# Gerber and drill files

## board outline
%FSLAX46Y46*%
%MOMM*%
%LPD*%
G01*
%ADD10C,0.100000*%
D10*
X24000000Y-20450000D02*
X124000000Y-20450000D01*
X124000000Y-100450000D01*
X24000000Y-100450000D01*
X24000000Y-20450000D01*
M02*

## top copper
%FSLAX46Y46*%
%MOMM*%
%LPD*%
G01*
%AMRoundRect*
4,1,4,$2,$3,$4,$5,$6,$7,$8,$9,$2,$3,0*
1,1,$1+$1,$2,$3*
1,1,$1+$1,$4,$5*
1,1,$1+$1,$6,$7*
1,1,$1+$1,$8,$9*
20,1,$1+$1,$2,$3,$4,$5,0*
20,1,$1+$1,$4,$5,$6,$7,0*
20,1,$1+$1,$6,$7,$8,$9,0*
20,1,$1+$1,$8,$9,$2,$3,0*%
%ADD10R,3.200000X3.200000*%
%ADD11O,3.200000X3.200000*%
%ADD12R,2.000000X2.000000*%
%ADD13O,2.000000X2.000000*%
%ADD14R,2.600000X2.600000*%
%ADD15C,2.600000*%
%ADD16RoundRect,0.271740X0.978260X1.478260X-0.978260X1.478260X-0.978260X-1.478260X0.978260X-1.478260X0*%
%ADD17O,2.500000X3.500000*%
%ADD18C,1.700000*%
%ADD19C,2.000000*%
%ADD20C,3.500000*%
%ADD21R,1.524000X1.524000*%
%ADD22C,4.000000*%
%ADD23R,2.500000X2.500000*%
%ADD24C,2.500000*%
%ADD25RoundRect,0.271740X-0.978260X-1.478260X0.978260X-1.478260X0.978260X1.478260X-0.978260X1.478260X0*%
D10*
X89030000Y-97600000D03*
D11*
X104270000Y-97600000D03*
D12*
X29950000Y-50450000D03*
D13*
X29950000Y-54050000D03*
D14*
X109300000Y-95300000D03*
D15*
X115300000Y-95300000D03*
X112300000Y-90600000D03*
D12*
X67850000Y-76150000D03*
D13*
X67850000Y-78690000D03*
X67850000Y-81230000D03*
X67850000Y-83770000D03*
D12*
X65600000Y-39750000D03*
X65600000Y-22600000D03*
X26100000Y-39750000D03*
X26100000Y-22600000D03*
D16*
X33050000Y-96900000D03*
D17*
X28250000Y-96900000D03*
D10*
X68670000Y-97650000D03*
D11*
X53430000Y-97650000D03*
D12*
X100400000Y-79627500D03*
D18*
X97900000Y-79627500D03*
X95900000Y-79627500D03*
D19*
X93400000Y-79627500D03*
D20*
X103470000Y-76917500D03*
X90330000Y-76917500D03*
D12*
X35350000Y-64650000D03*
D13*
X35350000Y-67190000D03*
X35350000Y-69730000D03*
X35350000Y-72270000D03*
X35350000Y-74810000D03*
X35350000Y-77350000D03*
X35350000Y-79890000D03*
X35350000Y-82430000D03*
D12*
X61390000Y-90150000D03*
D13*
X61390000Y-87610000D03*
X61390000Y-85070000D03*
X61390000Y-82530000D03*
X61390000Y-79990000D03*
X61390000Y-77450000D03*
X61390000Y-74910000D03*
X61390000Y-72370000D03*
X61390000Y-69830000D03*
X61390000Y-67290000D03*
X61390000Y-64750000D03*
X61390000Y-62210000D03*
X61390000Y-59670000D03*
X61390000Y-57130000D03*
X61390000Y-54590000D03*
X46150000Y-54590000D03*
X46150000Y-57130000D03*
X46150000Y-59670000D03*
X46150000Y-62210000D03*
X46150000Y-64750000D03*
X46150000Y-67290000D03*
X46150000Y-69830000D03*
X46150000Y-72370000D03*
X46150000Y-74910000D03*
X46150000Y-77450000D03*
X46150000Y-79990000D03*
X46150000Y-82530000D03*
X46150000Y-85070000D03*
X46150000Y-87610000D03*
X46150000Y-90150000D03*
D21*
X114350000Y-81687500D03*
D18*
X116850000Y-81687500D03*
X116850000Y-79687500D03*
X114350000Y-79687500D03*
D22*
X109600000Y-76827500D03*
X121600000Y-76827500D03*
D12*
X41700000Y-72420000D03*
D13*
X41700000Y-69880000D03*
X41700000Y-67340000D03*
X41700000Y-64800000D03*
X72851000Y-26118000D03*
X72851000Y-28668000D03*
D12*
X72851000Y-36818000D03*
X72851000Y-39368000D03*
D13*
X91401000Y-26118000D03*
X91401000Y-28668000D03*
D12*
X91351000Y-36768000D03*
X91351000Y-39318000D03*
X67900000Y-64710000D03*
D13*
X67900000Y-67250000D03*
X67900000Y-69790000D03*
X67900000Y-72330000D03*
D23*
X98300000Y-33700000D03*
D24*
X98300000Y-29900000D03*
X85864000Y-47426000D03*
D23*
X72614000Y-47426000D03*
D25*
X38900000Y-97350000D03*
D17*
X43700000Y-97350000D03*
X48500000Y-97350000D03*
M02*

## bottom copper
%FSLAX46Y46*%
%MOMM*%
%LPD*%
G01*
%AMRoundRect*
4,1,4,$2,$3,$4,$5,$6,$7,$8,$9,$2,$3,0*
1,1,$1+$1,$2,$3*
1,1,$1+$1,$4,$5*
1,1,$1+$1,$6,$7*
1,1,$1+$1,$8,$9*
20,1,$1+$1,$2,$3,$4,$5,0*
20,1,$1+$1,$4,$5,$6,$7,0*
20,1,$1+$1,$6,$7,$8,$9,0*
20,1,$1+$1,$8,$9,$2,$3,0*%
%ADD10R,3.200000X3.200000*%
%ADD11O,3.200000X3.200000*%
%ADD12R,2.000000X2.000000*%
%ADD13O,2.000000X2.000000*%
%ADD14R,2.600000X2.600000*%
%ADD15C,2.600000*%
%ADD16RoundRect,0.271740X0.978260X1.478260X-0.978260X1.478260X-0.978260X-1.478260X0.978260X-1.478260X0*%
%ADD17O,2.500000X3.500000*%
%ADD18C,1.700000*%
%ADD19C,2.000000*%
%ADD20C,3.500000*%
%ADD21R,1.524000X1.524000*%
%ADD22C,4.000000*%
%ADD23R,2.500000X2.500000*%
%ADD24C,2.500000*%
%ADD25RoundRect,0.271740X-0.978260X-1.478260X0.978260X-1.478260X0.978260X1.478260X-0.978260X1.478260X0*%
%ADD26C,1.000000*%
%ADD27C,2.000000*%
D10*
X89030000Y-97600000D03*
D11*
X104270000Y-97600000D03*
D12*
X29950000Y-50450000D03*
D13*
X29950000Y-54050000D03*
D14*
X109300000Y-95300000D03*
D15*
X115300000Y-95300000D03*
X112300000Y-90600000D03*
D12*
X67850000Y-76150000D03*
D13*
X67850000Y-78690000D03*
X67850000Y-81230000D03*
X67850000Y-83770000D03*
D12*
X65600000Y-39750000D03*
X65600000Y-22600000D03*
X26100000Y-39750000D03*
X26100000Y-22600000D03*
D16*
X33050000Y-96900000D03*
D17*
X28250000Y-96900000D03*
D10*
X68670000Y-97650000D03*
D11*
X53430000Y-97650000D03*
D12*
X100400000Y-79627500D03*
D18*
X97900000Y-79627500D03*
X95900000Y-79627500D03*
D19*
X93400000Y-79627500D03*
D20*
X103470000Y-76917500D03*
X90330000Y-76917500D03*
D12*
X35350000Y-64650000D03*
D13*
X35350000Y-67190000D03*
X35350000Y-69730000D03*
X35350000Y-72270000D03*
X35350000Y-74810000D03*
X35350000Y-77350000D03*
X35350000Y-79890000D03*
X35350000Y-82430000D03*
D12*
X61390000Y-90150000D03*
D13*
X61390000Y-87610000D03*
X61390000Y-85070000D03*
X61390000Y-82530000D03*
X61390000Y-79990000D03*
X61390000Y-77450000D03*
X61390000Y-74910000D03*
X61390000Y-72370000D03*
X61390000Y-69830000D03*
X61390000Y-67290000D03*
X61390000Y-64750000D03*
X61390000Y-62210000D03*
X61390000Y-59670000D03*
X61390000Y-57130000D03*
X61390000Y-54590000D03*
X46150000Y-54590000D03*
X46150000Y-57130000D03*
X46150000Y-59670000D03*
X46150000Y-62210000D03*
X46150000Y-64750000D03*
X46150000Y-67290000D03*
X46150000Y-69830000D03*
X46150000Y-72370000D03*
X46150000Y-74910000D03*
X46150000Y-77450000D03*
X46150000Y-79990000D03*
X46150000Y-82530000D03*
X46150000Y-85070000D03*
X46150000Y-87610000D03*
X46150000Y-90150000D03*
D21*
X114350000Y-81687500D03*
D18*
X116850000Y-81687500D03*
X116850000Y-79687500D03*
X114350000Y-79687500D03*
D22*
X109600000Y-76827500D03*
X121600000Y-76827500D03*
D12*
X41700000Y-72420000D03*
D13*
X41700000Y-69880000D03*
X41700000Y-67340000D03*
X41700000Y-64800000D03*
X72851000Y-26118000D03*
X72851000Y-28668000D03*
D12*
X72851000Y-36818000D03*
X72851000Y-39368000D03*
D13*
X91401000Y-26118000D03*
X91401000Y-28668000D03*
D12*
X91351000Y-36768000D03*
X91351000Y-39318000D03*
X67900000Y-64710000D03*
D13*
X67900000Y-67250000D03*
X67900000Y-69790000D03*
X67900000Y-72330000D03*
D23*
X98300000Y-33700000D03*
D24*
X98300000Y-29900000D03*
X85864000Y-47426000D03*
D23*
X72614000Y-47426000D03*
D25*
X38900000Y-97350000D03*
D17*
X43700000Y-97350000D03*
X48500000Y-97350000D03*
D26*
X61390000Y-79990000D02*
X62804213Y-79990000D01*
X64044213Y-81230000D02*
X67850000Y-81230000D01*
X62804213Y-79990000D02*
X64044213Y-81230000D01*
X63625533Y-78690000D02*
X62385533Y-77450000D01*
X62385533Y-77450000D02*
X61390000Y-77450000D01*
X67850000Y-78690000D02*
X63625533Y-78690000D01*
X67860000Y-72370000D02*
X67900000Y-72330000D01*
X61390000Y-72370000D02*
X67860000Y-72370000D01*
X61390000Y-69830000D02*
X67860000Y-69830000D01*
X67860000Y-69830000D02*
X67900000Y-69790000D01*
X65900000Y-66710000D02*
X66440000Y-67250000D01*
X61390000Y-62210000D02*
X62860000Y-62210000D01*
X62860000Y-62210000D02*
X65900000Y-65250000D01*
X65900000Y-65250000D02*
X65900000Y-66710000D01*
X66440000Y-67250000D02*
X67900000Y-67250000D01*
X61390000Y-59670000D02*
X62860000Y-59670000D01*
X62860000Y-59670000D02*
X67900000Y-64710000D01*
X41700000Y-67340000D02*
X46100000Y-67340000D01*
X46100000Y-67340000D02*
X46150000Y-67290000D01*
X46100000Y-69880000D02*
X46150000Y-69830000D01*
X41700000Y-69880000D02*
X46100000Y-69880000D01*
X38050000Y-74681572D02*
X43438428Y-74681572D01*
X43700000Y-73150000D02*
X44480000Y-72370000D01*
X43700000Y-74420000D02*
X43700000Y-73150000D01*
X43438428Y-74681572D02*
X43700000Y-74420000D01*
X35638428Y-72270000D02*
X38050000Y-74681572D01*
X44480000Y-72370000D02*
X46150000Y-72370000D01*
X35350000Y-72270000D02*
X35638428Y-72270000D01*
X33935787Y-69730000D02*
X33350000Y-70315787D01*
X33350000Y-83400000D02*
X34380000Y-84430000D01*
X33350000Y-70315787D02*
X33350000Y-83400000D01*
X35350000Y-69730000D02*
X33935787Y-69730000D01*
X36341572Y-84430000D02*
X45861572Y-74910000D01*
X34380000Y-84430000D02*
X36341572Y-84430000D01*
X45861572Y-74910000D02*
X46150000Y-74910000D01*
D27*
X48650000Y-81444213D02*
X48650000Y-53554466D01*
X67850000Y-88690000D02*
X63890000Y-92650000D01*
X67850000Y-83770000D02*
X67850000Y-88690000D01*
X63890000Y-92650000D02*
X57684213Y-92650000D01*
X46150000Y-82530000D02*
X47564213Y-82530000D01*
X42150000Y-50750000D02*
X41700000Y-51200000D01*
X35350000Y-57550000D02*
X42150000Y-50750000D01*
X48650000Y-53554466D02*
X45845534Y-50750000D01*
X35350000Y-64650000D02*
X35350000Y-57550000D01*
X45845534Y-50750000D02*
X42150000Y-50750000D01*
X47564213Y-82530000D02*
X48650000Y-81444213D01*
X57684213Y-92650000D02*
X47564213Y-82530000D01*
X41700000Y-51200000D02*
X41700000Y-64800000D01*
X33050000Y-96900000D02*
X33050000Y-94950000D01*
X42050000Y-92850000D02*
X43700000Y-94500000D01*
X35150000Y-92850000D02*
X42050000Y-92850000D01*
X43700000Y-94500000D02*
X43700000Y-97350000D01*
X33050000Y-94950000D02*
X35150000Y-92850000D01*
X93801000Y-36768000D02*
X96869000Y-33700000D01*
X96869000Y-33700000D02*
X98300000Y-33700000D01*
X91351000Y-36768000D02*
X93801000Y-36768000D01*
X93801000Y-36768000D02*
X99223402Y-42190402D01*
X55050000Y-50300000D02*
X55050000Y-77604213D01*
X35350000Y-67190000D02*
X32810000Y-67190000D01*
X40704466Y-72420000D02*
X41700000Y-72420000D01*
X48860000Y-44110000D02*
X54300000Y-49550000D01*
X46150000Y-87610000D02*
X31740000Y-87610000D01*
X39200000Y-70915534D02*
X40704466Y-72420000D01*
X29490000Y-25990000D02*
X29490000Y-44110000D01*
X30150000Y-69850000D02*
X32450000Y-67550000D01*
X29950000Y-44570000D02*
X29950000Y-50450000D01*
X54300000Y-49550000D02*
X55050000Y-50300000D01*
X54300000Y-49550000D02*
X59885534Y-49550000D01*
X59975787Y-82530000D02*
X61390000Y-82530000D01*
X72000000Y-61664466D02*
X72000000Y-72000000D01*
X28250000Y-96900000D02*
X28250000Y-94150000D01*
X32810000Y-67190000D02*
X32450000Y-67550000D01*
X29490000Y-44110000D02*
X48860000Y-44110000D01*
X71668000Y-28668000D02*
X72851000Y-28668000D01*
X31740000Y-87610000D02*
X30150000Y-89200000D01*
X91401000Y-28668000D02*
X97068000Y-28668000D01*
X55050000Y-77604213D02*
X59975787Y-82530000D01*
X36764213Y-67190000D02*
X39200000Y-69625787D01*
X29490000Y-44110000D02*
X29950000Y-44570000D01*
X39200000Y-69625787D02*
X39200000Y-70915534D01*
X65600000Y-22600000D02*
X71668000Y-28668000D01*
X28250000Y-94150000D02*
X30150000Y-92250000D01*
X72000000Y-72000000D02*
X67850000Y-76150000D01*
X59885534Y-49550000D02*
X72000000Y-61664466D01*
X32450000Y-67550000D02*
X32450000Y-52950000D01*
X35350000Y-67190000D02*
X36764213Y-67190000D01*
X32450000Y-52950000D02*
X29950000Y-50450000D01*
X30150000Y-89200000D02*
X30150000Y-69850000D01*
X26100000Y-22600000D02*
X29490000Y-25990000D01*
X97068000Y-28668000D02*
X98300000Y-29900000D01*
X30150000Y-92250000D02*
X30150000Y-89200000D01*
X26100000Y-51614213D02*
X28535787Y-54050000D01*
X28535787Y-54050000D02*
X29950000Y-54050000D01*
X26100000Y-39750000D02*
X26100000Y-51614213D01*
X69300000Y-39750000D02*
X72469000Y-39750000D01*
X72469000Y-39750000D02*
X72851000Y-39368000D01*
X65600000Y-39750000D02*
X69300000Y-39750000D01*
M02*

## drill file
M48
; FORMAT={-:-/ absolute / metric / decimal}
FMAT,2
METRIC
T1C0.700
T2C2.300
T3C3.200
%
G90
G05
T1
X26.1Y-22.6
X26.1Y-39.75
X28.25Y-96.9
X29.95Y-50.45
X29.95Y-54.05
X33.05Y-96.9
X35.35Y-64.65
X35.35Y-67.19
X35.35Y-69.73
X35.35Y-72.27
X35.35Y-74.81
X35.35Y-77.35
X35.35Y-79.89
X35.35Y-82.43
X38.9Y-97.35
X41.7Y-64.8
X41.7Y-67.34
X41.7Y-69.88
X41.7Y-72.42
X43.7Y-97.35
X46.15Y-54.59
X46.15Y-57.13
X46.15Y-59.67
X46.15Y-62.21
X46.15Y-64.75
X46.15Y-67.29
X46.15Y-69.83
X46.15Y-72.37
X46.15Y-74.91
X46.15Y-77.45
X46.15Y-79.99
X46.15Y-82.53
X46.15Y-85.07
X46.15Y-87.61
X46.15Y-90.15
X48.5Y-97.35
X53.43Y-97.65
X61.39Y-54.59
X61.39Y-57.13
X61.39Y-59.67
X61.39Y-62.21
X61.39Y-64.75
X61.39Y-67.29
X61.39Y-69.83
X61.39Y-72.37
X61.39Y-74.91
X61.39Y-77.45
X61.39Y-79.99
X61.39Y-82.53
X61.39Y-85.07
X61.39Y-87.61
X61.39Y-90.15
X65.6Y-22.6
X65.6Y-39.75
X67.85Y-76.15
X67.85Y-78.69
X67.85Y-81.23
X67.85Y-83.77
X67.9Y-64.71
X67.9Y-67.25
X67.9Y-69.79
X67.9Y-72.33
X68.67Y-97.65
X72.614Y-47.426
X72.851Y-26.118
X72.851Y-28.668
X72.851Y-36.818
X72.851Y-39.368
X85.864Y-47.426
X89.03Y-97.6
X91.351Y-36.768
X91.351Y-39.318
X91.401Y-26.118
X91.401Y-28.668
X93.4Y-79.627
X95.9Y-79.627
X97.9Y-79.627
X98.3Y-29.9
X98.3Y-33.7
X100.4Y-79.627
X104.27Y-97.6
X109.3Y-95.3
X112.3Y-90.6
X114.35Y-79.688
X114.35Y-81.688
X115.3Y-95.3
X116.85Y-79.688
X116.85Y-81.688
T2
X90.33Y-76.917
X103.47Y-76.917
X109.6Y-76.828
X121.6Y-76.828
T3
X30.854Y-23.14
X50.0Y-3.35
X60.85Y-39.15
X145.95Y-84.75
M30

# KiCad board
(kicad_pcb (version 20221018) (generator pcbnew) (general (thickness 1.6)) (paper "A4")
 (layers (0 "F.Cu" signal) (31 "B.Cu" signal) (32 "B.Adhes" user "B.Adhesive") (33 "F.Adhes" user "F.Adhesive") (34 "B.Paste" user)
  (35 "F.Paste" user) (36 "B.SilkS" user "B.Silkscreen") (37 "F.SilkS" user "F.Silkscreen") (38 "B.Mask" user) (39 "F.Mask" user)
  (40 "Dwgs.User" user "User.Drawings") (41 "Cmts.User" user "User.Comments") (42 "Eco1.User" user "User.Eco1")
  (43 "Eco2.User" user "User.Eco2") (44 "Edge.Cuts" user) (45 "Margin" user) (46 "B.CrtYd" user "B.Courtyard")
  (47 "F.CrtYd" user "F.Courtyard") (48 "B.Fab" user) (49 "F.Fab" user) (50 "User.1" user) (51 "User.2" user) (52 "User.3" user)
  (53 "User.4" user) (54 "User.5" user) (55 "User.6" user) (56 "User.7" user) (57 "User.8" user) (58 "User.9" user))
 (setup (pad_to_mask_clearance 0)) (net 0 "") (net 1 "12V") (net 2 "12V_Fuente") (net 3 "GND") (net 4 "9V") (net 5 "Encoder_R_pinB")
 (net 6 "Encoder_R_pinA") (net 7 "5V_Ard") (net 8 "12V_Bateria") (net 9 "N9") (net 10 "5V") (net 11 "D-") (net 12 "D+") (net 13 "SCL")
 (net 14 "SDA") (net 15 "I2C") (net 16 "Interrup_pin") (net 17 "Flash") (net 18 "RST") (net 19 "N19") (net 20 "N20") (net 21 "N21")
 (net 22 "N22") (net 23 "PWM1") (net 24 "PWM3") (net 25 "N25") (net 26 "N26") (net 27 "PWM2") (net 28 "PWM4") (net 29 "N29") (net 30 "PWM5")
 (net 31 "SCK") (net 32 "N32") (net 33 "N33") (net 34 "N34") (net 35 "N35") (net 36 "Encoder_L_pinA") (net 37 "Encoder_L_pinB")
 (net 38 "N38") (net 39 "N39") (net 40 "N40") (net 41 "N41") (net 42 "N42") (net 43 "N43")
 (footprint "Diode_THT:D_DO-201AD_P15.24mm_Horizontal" (layer "F.Cu") (at 89.03 97.6)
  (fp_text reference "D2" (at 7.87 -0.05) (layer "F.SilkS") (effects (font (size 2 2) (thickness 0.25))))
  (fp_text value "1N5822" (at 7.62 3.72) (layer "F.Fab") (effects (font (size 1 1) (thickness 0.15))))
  (pad "1" thru_hole rect (at 0 0) (size 3.2 3.2) (drill 0.7) (layers "*.Cu" "*.Mask") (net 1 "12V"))
  (pad "2" thru_hole oval (at 15.24 0) (size 3.2 3.2) (drill 0.7) (layers "*.Cu" "*.Mask") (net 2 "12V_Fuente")))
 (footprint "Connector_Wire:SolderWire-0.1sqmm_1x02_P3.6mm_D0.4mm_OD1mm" (layer "F.Cu") (at 29.95 50.45 -90)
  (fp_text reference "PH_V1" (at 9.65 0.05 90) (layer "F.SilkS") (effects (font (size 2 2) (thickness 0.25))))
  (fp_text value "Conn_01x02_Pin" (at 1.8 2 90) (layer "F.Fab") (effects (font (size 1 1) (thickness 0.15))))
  (pad "1" thru_hole rect (at 0 0 270) (size 2 2) (drill 0.7) (layers "*.Cu" "*.Mask") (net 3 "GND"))
  (pad "2" thru_hole oval (at 3.6 0 270) (size 2 2) (drill 0.7) (layers "*.Cu" "*.Mask") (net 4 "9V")))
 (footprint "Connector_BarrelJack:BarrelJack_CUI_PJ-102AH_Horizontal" (layer "F.Cu") (at 109.3 95.3 90)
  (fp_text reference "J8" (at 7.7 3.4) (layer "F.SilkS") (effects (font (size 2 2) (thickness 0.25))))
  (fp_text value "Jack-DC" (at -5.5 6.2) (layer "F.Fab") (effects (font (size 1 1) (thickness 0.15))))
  (pad "1" thru_hole rect (at 0 0 90) (size 2.6 2.6) (drill 0.7) (layers "*.Cu" "*.Mask") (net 2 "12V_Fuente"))
  (pad "2" thru_hole circle (at 0 6 90) (size 2.6 2.6) (drill 0.7) (layers "*.Cu" "*.Mask") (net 3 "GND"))
  (pad "3" thru_hole circle (at 4.7 3 90) (size 2.6 2.6) (drill 0.7) (layers "*.Cu" "*.Mask")))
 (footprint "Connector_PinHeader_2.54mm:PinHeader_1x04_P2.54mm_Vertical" (layer "F.Cu") (at 67.85 76.15)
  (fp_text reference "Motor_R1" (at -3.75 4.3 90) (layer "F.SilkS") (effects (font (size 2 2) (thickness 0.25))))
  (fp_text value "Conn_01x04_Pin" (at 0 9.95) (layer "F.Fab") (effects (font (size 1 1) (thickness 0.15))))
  (pad "1" thru_hole rect (at 0 0) (size 2 2) (drill 0.7) (layers "*.Cu" "*.Mask") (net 3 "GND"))
  (pad "2" thru_hole oval (at 0 2.54) (size 2 2) (drill 0.7) (layers "*.Cu" "*.Mask") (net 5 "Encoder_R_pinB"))
  (pad "3" thru_hole oval (at 0 5.08) (size 2 2) (drill 0.7) (layers "*.Cu" "*.Mask") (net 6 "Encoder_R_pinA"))
  (pad "4" thru_hole oval (at 0 7.62) (size 2 2) (drill 0.7) (layers "*.Cu" "*.Mask") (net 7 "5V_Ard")))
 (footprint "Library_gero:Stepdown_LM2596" (layer "F.Cu") (at 67.45 41.7 180)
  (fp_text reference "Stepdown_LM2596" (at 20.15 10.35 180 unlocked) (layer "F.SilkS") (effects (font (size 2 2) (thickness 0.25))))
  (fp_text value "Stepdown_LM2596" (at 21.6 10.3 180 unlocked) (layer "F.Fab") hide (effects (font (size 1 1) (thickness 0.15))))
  (pad "" np_thru_hole circle (at 6.6 2.55 180) (size 3.2 3.2) (drill 3.2) (layers "F&B.Cu" "*.Mask") (thermal_bridge_angle 90))
  (pad "" np_thru_hole circle (at 36.596 18.56 180) (size 3.2 3.2) (drill 3.2) (layers "F&B.Cu" "*.Mask") (thermal_bridge_angle 90))
  (pad "1" thru_hole rect (at 1.85 1.95 180) (size 2 2) (drill 0.7) (layers "*.Cu" "*.Mask") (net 1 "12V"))
  (pad "2" thru_hole rect (at 1.85 19.1 180) (size 2 2) (drill 0.7) (layers "*.Cu" "*.Mask") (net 3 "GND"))
  (pad "3" thru_hole rect (at 41.35 1.95 180) (size 2 2) (drill 0.7) (layers "*.Cu" "*.Mask") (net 4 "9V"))
  (pad "4" thru_hole rect (at 41.35 19.1 180) (size 2 2) (drill 0.7) (layers "*.Cu" "*.Mask") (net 3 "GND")))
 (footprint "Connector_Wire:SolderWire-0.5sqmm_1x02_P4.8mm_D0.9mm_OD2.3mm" (layer "F.Cu") (at 33.05 96.9 180)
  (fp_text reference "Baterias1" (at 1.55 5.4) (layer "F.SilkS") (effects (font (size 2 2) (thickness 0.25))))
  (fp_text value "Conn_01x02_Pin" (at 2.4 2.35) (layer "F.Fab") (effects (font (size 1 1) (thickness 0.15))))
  (pad "1" thru_hole roundrect (at 0 0 180) (size 2.5 3.5) (drill 0.7) (layers "*.Cu" "*.Mask") (roundrect_rratio 0.108696)
   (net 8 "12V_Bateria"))
  (pad "2" thru_hole oval (at 4.8 0 180) (size 2.5 3.5) (drill 0.7) (layers "*.Cu" "*.Mask") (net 3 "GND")))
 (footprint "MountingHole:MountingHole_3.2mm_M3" (layer "F.Cu") (at 50 3.35)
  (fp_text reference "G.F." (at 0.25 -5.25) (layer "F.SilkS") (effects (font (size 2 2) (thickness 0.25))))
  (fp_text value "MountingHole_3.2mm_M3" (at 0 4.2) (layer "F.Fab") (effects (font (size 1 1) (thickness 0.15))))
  (pad "" np_thru_hole circle (at 0 0) (size 3.2 3.2) (drill 3.2) (layers "F&B.Cu" "*.Mask")))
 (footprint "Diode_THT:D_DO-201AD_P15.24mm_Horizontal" (layer "F.Cu") (at 68.67 97.65 180)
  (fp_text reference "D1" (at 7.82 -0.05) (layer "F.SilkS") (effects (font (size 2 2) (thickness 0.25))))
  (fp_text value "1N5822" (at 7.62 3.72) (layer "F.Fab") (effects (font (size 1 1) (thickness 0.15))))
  (pad "1" thru_hole rect (at 0 0 180) (size 3.2 3.2) (drill 0.7) (layers "*.Cu" "*.Mask") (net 1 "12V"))
  (pad "2" thru_hole oval (at 15.24 0 180) (size 3.2 3.2) (drill 0.7) (layers "*.Cu" "*.Mask") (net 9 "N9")))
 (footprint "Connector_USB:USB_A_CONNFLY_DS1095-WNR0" (layer "F.Cu") (at 100.4 79.6275 180)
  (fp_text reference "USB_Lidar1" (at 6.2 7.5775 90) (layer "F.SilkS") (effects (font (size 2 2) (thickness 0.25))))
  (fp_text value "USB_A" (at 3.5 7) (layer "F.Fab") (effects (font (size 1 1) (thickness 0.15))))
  (pad "1" thru_hole rect (at 0 0 180) (size 2 2) (drill 0.7) (layers "*.Cu" "*.Mask") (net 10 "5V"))
  (pad "2" thru_hole circle (at 2.5 0 180) (size 1.7 1.7) (drill 0.7) (layers "*.Cu" "*.Mask") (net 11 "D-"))
  (pad "3" thru_hole circle (at 4.5 0 180) (size 1.7 1.7) (drill 0.7) (layers "*.Cu" "*.Mask") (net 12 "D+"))
  (pad "4" thru_hole circle (at 7 0 180) (size 2 2) (drill 0.7) (layers "*.Cu" "*.Mask") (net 3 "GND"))
  (pad "5" thru_hole circle (at -3.07 2.71 180) (size 3.5 3.5) (drill 2.3) (layers "*.Cu" "*.Mask") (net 3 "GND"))
  (pad "5" thru_hole circle (at 10.07 2.71 180) (size 3.5 3.5) (drill 2.3) (layers "*.Cu" "*.Mask") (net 3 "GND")))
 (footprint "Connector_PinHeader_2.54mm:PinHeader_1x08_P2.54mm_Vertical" (layer "F.Cu") (at 35.35 64.65)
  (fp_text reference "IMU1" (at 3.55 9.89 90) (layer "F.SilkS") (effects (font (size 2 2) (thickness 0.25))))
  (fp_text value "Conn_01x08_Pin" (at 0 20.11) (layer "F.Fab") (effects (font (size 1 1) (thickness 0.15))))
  (pad "1" thru_hole rect (at 0 0) (size 2 2) (drill 0.7) (layers "*.Cu" "*.Mask") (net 7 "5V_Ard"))
  (pad "2" thru_hole oval (at 0 2.54) (size 2 2) (drill 0.7) (layers "*.Cu" "*.Mask") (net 3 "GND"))
  (pad "3" thru_hole oval (at 0 5.08) (size 2 2) (drill 0.7) (layers "*.Cu" "*.Mask") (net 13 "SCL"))
  (pad "4" thru_hole oval (at 0 7.62) (size 2 2) (drill 0.7) (layers "*.Cu" "*.Mask") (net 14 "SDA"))
  (pad "5" thru_hole oval (at 0 10.16) (size 2 2) (drill 0.7) (layers "*.Cu" "*.Mask") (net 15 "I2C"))
  (pad "6" thru_hole oval (at 0 12.7) (size 2 2) (drill 0.7) (layers "*.Cu" "*.Mask") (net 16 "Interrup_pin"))
  (pad "7" thru_hole oval (at 0 15.24) (size 2 2) (drill 0.7) (layers "*.Cu" "*.Mask") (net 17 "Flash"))
  (pad "8" thru_hole oval (at 0 17.78) (size 2 2) (drill 0.7) (layers "*.Cu" "*.Mask") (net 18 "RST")))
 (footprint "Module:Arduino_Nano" (layer "F.Cu") (at 61.39 90.15 180)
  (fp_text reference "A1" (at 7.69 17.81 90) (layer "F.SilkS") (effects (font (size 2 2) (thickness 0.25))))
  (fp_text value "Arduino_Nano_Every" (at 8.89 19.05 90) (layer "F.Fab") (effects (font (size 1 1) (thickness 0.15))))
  (pad "1" thru_hole rect (at 0 0 180) (size 2 2) (drill 0.7) (layers "*.Cu" "*.Mask") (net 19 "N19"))
  (pad "2" thru_hole oval (at 0 2.54 180) (size 2 2) (drill 0.7) (layers "*.Cu" "*.Mask") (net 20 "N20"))
  (pad "3" thru_hole oval (at 0 5.08 180) (size 2 2) (drill 0.7) (layers "*.Cu" "*.Mask") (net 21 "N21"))
  (pad "4" thru_hole oval (at 0 7.62 180) (size 2 2) (drill 0.7) (layers "*.Cu" "*.Mask") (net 3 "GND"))
  (pad "5" thru_hole oval (at 0 10.16 180) (size 2 2) (drill 0.7) (layers "*.Cu" "*.Mask") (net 6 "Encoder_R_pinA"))
  (pad "6" thru_hole oval (at 0 12.7 180) (size 2 2) (drill 0.7) (layers "*.Cu" "*.Mask") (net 5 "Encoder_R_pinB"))
  (pad "7" thru_hole oval (at 0 15.24 180) (size 2 2) (drill 0.7) (layers "*.Cu" "*.Mask") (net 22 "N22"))
  (pad "8" thru_hole oval (at 0 17.78 180) (size 2 2) (drill 0.7) (layers "*.Cu" "*.Mask") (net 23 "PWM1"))
  (pad "9" thru_hole oval (at 0 20.32 180) (size 2 2) (drill 0.7) (layers "*.Cu" "*.Mask") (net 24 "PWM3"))
  (pad "10" thru_hole oval (at 0 22.86 180) (size 2 2) (drill 0.7) (layers "*.Cu" "*.Mask") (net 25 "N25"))
  (pad "11" thru_hole oval (at 0 25.4 180) (size 2 2) (drill 0.7) (layers "*.Cu" "*.Mask") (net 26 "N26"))
  (pad "12" thru_hole oval (at 0 27.94 180) (size 2 2) (drill 0.7) (layers "*.Cu" "*.Mask") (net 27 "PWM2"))
  (pad "13" thru_hole oval (at 0 30.48 180) (size 2 2) (drill 0.7) (layers "*.Cu" "*.Mask") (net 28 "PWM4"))
  (pad "14" thru_hole oval (at 0 33.02 180) (size 2 2) (drill 0.7) (layers "*.Cu" "*.Mask") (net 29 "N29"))
  (pad "15" thru_hole oval (at 0 35.56 180) (size 2 2) (drill 0.7) (layers "*.Cu" "*.Mask") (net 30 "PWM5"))
  (pad "16" thru_hole oval (at 15.24 35.56 180) (size 2 2) (drill 0.7) (layers "*.Cu" "*.Mask") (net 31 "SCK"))
  (pad "17" thru_hole oval (at 15.24 33.02 180) (size 2 2) (drill 0.7) (layers "*.Cu" "*.Mask") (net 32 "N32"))
  (pad "18" thru_hole oval (at 15.24 30.48 180) (size 2 2) (drill 0.7) (layers "*.Cu" "*.Mask") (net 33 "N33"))
  (pad "19" thru_hole oval (at 15.24 27.94 180) (size 2 2) (drill 0.7) (layers "*.Cu" "*.Mask") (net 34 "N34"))
  (pad "20" thru_hole oval (at 15.24 25.4 180) (size 2 2) (drill 0.7) (layers "*.Cu" "*.Mask") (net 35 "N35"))
  (pad "21" thru_hole oval (at 15.24 22.86 180) (size 2 2) (drill 0.7) (layers "*.Cu" "*.Mask") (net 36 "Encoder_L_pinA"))
  (pad "22" thru_hole oval (at 15.24 20.32 180) (size 2 2) (drill 0.7) (layers "*.Cu" "*.Mask") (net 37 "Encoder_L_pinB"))
  (pad "23" thru_hole oval (at 15.24 17.78 180) (size 2 2) (drill 0.7) (layers "*.Cu" "*.Mask") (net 14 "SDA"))
  (pad "24" thru_hole oval (at 15.24 15.24 180) (size 2 2) (drill 0.7) (layers "*.Cu" "*.Mask") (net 13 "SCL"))
  (pad "25" thru_hole oval (at 15.24 12.7 180) (size 2 2) (drill 0.7) (layers "*.Cu" "*.Mask") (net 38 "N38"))
  (pad "26" thru_hole oval (at 15.24 10.16 180) (size 2 2) (drill 0.7) (layers "*.Cu" "*.Mask") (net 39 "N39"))
  (pad "27" thru_hole oval (at 15.24 7.62 180) (size 2 2) (drill 0.7) (layers "*.Cu" "*.Mask") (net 7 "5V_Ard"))
  (pad "28" thru_hole oval (at 15.24 5.08 180) (size 2 2) (drill 0.7) (layers "*.Cu" "*.Mask") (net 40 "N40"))
  (pad "29" thru_hole oval (at 15.24 2.54 180) (size 2 2) (drill 0.7) (layers "*.Cu" "*.Mask") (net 3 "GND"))
  (pad "30" thru_hole oval (at 15.24 0 180) (size 2 2) (drill 0.7) (layers "*.Cu" "*.Mask") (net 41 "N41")))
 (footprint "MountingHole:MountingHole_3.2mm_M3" (layer "F.Cu") (at 145.95 84.75)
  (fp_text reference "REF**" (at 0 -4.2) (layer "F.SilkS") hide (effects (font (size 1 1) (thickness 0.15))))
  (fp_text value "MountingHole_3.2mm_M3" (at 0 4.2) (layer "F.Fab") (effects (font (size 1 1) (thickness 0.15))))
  (pad "" np_thru_hole circle (at 0 0) (size 3.2 3.2) (drill 3.2) (layers "*.Cu" "*.Mask")))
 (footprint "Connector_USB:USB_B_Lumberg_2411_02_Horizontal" (layer "F.Cu") (at 114.35 81.6875 90)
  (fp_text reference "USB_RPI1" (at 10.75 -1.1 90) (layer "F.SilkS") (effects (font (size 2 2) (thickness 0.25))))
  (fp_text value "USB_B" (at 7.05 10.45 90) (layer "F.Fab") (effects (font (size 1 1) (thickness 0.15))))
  (pad "1" thru_hole rect (at 0 0 90) (size 1.524 1.524) (drill 0.7) (layers "*.Cu" "*.Mask") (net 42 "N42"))
  (pad "2" thru_hole circle (at 0 2.5 90) (size 1.7 1.7) (drill 0.7) (layers "*.Cu" "*.Mask") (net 11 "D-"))
  (pad "3" thru_hole circle (at 2 2.5 90) (size 1.7 1.7) (drill 0.7) (layers "*.Cu" "*.Mask") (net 12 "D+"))
  (pad "4" thru_hole circle (at 2 0 90) (size 1.7 1.7) (drill 0.7) (layers "*.Cu" "*.Mask") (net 3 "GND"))
  (pad "5" thru_hole circle (at 4.86 -4.75 180) (size 4 4) (drill 2.3) (layers "*.Cu" "*.Mask") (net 3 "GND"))
  (pad "5" thru_hole circle (at 4.86 7.25 180) (size 4 4) (drill 2.3) (layers "*.Cu" "*.Mask") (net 3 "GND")))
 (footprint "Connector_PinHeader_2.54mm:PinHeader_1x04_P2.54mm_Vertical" (layer "F.Cu") (at 41.7 72.42 180)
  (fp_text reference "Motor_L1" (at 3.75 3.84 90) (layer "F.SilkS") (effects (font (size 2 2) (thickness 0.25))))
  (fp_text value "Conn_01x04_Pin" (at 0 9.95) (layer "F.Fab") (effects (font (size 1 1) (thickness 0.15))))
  (pad "1" thru_hole rect (at 0 0 180) (size 2 2) (drill 0.7) (layers "*.Cu" "*.Mask") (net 3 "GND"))
  (pad "2" thru_hole oval (at 0 2.54 180) (size 2 2) (drill 0.7) (layers "*.Cu" "*.Mask") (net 37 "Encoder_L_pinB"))
  (pad "3" thru_hole oval (at 0 5.08 180) (size 2 2) (drill 0.7) (layers "*.Cu" "*.Mask") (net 36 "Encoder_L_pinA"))
  (pad "4" thru_hole oval (at 0 7.62 180) (size 2 2) (drill 0.7) (layers "*.Cu" "*.Mask") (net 7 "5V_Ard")))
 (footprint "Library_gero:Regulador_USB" (layer "F.Cu") (at 71.051 24.368)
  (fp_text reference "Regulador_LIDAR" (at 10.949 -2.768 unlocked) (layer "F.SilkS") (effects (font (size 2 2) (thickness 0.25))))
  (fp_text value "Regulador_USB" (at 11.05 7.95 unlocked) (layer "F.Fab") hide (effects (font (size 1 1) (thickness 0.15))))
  (pad "1" thru_hole oval (at 1.8 1.75) (size 2 2) (drill 0.7) (layers "*.Cu" "*.Mask"))
  (pad "2" thru_hole oval (at 1.8 4.3) (size 2 2) (drill 0.7) (layers "*.Cu" "*.Mask") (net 3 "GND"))
  (pad "3" thru_hole rect (at 1.8 12.45) (size 2 2) (drill 0.7) (layers "*.Cu" "*.Mask") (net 1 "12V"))
  (pad "4" thru_hole rect (at 1.8 15) (size 2 2) (drill 0.7) (layers "*.Cu" "*.Mask") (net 1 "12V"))
  (pad "5" thru_hole oval (at 20.35 1.75) (size 2 2) (drill 0.7) (layers "*.Cu" "*.Mask"))
  (pad "6" thru_hole oval (at 20.35 4.3) (size 2 2) (drill 0.7) (layers "*.Cu" "*.Mask") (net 3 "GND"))
  (pad "7" thru_hole rect (at 20.3 12.4) (size 2 2) (drill 0.7) (layers "*.Cu" "*.Mask") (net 10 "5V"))
  (pad "8" thru_hole rect (at 20.3 14.95) (size 2 2) (drill 0.7) (layers "*.Cu" "*.Mask")))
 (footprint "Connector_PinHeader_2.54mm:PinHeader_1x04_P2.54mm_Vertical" (layer "F.Cu") (at 67.9 64.71)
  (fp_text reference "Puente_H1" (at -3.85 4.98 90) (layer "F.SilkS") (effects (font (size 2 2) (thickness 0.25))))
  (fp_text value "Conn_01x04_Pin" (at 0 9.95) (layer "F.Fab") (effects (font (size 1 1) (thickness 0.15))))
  (pad "1" thru_hole rect (at 0 0) (size 2 2) (drill 0.7) (layers "*.Cu" "*.Mask") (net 28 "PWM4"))
  (pad "2" thru_hole oval (at 0 2.54) (size 2 2) (drill 0.7) (layers "*.Cu" "*.Mask") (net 27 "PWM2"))
  (pad "3" thru_hole oval (at 0 5.08) (size 2 2) (drill 0.7) (layers "*.Cu" "*.Mask") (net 24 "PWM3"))
  (pad "4" thru_hole oval (at 0 7.62) (size 2 2) (drill 0.7) (layers "*.Cu" "*.Mask") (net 23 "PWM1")))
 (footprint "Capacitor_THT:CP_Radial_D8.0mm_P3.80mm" (layer "F.Cu") (at 98.3 33.7 90)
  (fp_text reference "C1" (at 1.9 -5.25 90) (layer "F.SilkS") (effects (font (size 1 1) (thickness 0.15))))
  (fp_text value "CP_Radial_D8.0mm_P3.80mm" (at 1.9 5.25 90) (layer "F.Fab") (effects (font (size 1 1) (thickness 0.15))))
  (pad "1" thru_hole rect (at 0 0 90) (size 2.5 2.5) (drill 0.7) (layers "*.Cu" "*.Mask") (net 10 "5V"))
  (pad "2" thru_hole circle (at 3.8 0 90) (size 2.5 2.5) (drill 0.7) (layers "*.Cu" "*.Mask") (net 3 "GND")))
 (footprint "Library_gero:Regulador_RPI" (layer "F.Cu") (at 92.4 45.124 -90)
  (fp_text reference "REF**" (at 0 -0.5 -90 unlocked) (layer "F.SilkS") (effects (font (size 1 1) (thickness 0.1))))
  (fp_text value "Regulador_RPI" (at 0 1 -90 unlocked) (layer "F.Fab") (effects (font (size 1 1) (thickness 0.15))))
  (pad "1" thru_hole circle (at 2.302 6.536 270) (size 2.5 2.5) (drill 0.7) (layers "*.Cu" "*.Mask") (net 3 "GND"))
  (pad "2" thru_hole rect (at 2.302 19.786 270) (size 2.5 2.5) (drill 0.7) (layers "*.Cu" "*.Mask") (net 1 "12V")))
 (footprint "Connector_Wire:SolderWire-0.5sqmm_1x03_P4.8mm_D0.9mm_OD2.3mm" (layer "F.Cu") (at 38.9 97.35)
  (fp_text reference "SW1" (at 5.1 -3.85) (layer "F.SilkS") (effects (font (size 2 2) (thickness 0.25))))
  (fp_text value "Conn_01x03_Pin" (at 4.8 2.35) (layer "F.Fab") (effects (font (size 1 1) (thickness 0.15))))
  (pad "1" thru_hole roundrect (at 0 0) (size 2.5 3.5) (drill 0.7) (layers "*.Cu" "*.Mask") (roundrect_rratio 0.108696) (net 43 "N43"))
  (pad "2" thru_hole oval (at 4.8 0) (size 2.5 3.5) (drill 0.7) (layers "*.Cu" "*.Mask") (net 8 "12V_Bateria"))
  (pad "3" thru_hole oval (at 9.6 0) (size 2.5 3.5) (drill 0.7) (layers "*.Cu" "*.Mask") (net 9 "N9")))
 (gr_rect (start 24 20.45) (end 124 100.45) (stroke (width 0.1) (type default)) (fill none) (layer "Edge.Cuts"))
 (segment (start 61.39 79.99) (end 62.804213 79.99) (width 1) (layer "B.Cu") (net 6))
 (segment (start 64.044213 81.23) (end 67.85 81.23) (width 1) (layer "B.Cu") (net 6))
 (segment (start 62.804213 79.99) (end 64.044213 81.23) (width 1) (layer "B.Cu") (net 6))
 (segment (start 63.625533 78.69) (end 62.385533 77.45) (width 1) (layer "B.Cu") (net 5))
 (segment (start 62.385533 77.45) (end 61.39 77.45) (width 1) (layer "B.Cu") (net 5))
 (segment (start 67.85 78.69) (end 63.625533 78.69) (width 1) (layer "B.Cu") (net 5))
 (segment (start 67.86 72.37) (end 67.9 72.33) (width 1) (layer "B.Cu") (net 23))
 (segment (start 61.39 72.37) (end 67.86 72.37) (width 1) (layer "B.Cu") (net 23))
 (segment (start 61.39 69.83) (end 67.86 69.83) (width 1) (layer "B.Cu") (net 24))
 (segment (start 67.86 69.83) (end 67.9 69.79) (width 1) (layer "B.Cu") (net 24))
 (segment (start 65.9 66.71) (end 66.44 67.25) (width 1) (layer "B.Cu") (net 27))
 (segment (start 61.39 62.21) (end 62.86 62.21) (width 1) (layer "B.Cu") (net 27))
 (segment (start 62.86 62.21) (end 65.9 65.25) (width 1) (layer "B.Cu") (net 27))
 (segment (start 65.9 65.25) (end 65.9 66.71) (width 1) (layer "B.Cu") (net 27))
 (segment (start 66.44 67.25) (end 67.9 67.25) (width 1) (layer "B.Cu") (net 27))
 (segment (start 61.39 59.67) (end 62.86 59.67) (width 1) (layer "B.Cu") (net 28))
 (segment (start 62.86 59.67) (end 67.9 64.71) (width 1) (layer "B.Cu") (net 28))
 (segment (start 41.7 67.34) (end 46.1 67.34) (width 1) (layer "B.Cu") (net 36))
 (segment (start 46.1 67.34) (end 46.15 67.29) (width 1) (layer "B.Cu") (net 36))
 (segment (start 46.1 69.88) (end 46.15 69.83) (width 1) (layer "B.Cu") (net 37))
 (segment (start 41.7 69.88) (end 46.1 69.88) (width 1) (layer "B.Cu") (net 37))
 (segment (start 38.05 74.681572) (end 43.438428 74.681572) (width 1) (layer "B.Cu") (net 14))
 (segment (start 43.7 73.15) (end 44.48 72.37) (width 1) (layer "B.Cu") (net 14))
 (segment (start 43.7 74.42) (end 43.7 73.15) (width 1) (layer "B.Cu") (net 14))
 (segment (start 43.438428 74.681572) (end 43.7 74.42) (width 1) (layer "B.Cu") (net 14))
 (segment (start 35.638428 72.27) (end 38.05 74.681572) (width 1) (layer "B.Cu") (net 14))
 (segment (start 44.48 72.37) (end 46.15 72.37) (width 1) (layer "B.Cu") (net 14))
 (segment (start 35.35 72.27) (end 35.638428 72.27) (width 1) (layer "B.Cu") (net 14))
 (segment (start 33.935787 69.73) (end 33.35 70.315787) (width 1) (layer "B.Cu") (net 13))
 (segment (start 33.35 83.4) (end 34.38 84.43) (width 1) (layer "B.Cu") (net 13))
 (segment (start 33.35 70.315787) (end 33.35 83.4) (width 1) (layer "B.Cu") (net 13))
 (segment (start 35.35 69.73) (end 33.935787 69.73) (width 1) (layer "B.Cu") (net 13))
 (segment (start 36.341572 84.43) (end 45.861572 74.91) (width 1) (layer "B.Cu") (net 13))
 (segment (start 34.38 84.43) (end 36.341572 84.43) (width 1) (layer "B.Cu") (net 13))
 (segment (start 45.861572 74.91) (end 46.15 74.91) (width 1) (layer "B.Cu") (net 13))
 (segment (start 48.65 81.444213) (end 48.65 53.554466) (width 2) (layer "B.Cu") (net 7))
 (segment (start 67.85 88.69) (end 63.89 92.65) (width 2) (layer "B.Cu") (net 7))
 (segment (start 67.85 83.77) (end 67.85 88.69) (width 2) (layer "B.Cu") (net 7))
 (segment (start 63.89 92.65) (end 57.684213 92.65) (width 2) (layer "B.Cu") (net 7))
 (segment (start 46.15 82.53) (end 47.564213 82.53) (width 2) (layer "B.Cu") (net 7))
 (segment (start 42.15 50.75) (end 41.7 51.2) (width 2) (layer "B.Cu") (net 7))
 (segment (start 35.35 57.55) (end 42.15 50.75) (width 2) (layer "B.Cu") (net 7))
 (segment (start 48.65 53.554466) (end 45.845534 50.75) (width 2) (layer "B.Cu") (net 7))
 (segment (start 35.35 64.65) (end 35.35 57.55) (width 2) (layer "B.Cu") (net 7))
 (segment (start 45.845534 50.75) (end 42.15 50.75) (width 2) (layer "B.Cu") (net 7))
 (segment (start 47.564213 82.53) (end 48.65 81.444213) (width 2) (layer "B.Cu") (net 7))
 (segment (start 57.684213 92.65) (end 47.564213 82.53) (width 2) (layer "B.Cu") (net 7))
 (segment (start 41.7 51.2) (end 41.7 64.8) (width 2) (layer "B.Cu") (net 7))
 (segment (start 33.05 96.9) (end 33.05 94.95) (width 2) (layer "B.Cu") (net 8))
 (segment (start 42.05 92.85) (end 43.7 94.5) (width 2) (layer "B.Cu") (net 8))
 (segment (start 35.15 92.85) (end 42.05 92.85) (width 2) (layer "B.Cu") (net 8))
 (segment (start 43.7 94.5) (end 43.7 97.35) (width 2) (layer "B.Cu") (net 8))
 (segment (start 33.05 94.95) (end 35.15 92.85) (width 2) (layer "B.Cu") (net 8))
 (segment (start 93.801 36.768) (end 96.869 33.7) (width 2) (layer "B.Cu") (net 10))
 (segment (start 96.869 33.7) (end 98.3 33.7) (width 2) (layer "B.Cu") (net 10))
 (segment (start 91.351 36.768) (end 93.801 36.768) (width 2) (layer "B.Cu") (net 10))
 (segment (start 93.801 36.768) (end 99.223402 42.190402) (width 2) (layer "B.Cu") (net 10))
 (segment (start 55.05 50.3) (end 55.05 77.604213) (width 2) (layer "B.Cu") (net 3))
 (segment (start 35.35 67.19) (end 32.81 67.19) (width 2) (layer "B.Cu") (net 3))
 (segment (start 40.704466 72.42) (end 41.7 72.42) (width 2) (layer "B.Cu") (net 3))
 (segment (start 48.86 44.11) (end 54.3 49.55) (width 2) (layer "B.Cu") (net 3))
 (segment (start 46.15 87.61) (end 31.74 87.61) (width 2) (layer "B.Cu") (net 3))
 (segment (start 39.2 70.915534) (end 40.704466 72.42) (width 2) (layer "B.Cu") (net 3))
 (segment (start 29.49 25.99) (end 29.49 44.11) (width 2) (layer "B.Cu") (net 3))
 (segment (start 30.15 69.85) (end 32.45 67.55) (width 2) (layer "B.Cu") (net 3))
 (segment (start 29.95 44.57) (end 29.95 50.45) (width 2) (layer "B.Cu") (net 3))
 (segment (start 54.3 49.55) (end 55.05 50.3) (width 2) (layer "B.Cu") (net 3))
 (segment (start 54.3 49.55) (end 59.885534 49.55) (width 2) (layer "B.Cu") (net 3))
 (segment (start 59.975787 82.53) (end 61.39 82.53) (width 2) (layer "B.Cu") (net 3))
 (segment (start 72 61.664466) (end 72 72) (width 2) (layer "B.Cu") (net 3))
 (segment (start 28.25 96.9) (end 28.25 94.15) (width 2) (layer "B.Cu") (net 3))
 (segment (start 32.81 67.19) (end 32.45 67.55) (width 2) (layer "B.Cu") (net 3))
 (segment (start 29.49 44.11) (end 48.86 44.11) (width 2) (layer "B.Cu") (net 3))
 (segment (start 71.668 28.668) (end 72.851 28.668) (width 2) (layer "B.Cu") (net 3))
 (segment (start 31.74 87.61) (end 30.15 89.2) (width 2) (layer "B.Cu") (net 3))
 (segment (start 91.401 28.668) (end 97.068 28.668) (width 2) (layer "B.Cu") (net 3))
 (segment (start 55.05 77.604213) (end 59.975787 82.53) (width 2) (layer "B.Cu") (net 3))
 (segment (start 36.764213 67.19) (end 39.2 69.625787) (width 2) (layer "B.Cu") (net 3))
 (segment (start 29.49 44.11) (end 29.95 44.57) (width 2) (layer "B.Cu") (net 3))
 (segment (start 39.2 69.625787) (end 39.2 70.915534) (width 2) (layer "B.Cu") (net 3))
 (segment (start 65.6 22.6) (end 71.668 28.668) (width 2) (layer "B.Cu") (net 3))
 (segment (start 28.25 94.15) (end 30.15 92.25) (width 2) (layer "B.Cu") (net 3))
 (segment (start 72 72) (end 67.85 76.15) (width 2) (layer "B.Cu") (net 3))
 (segment (start 59.885534 49.55) (end 72 61.664466) (width 2) (layer "B.Cu") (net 3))
 (segment (start 32.45 67.55) (end 32.45 52.95) (width 2) (layer "B.Cu") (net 3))
 (segment (start 35.35 67.19) (end 36.764213 67.19) (width 2) (layer "B.Cu") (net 3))
 (segment (start 32.45 52.95) (end 29.95 50.45) (width 2) (layer "B.Cu") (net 3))
 (segment (start 30.15 89.2) (end 30.15 69.85) (width 2) (layer "B.Cu") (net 3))
 (segment (start 26.1 22.6) (end 29.49 25.99) (width 2) (layer "B.Cu") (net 3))
 (segment (start 97.068 28.668) (end 98.3 29.9) (width 2) (layer "B.Cu") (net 3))
 (segment (start 30.15 92.25) (end 30.15 89.2) (width 2) (layer "B.Cu") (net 3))
 (segment (start 26.1 51.614213) (end 28.535787 54.05) (width 2) (layer "B.Cu") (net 4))
 (segment (start 28.535787 54.05) (end 29.95 54.05) (width 2) (layer "B.Cu") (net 4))
 (segment (start 26.1 39.75) (end 26.1 51.614213) (width 2) (layer "B.Cu") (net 4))
 (segment (start 69.3 39.75) (end 72.469 39.75) (width 2) (layer "B.Cu") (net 1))
 (segment (start 72.469 39.75) (end 72.851 39.368) (width 2) (layer "B.Cu") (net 1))
 (segment (start 65.6 39.75) (end 69.3 39.75) (width 2) (layer "B.Cu") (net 1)))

